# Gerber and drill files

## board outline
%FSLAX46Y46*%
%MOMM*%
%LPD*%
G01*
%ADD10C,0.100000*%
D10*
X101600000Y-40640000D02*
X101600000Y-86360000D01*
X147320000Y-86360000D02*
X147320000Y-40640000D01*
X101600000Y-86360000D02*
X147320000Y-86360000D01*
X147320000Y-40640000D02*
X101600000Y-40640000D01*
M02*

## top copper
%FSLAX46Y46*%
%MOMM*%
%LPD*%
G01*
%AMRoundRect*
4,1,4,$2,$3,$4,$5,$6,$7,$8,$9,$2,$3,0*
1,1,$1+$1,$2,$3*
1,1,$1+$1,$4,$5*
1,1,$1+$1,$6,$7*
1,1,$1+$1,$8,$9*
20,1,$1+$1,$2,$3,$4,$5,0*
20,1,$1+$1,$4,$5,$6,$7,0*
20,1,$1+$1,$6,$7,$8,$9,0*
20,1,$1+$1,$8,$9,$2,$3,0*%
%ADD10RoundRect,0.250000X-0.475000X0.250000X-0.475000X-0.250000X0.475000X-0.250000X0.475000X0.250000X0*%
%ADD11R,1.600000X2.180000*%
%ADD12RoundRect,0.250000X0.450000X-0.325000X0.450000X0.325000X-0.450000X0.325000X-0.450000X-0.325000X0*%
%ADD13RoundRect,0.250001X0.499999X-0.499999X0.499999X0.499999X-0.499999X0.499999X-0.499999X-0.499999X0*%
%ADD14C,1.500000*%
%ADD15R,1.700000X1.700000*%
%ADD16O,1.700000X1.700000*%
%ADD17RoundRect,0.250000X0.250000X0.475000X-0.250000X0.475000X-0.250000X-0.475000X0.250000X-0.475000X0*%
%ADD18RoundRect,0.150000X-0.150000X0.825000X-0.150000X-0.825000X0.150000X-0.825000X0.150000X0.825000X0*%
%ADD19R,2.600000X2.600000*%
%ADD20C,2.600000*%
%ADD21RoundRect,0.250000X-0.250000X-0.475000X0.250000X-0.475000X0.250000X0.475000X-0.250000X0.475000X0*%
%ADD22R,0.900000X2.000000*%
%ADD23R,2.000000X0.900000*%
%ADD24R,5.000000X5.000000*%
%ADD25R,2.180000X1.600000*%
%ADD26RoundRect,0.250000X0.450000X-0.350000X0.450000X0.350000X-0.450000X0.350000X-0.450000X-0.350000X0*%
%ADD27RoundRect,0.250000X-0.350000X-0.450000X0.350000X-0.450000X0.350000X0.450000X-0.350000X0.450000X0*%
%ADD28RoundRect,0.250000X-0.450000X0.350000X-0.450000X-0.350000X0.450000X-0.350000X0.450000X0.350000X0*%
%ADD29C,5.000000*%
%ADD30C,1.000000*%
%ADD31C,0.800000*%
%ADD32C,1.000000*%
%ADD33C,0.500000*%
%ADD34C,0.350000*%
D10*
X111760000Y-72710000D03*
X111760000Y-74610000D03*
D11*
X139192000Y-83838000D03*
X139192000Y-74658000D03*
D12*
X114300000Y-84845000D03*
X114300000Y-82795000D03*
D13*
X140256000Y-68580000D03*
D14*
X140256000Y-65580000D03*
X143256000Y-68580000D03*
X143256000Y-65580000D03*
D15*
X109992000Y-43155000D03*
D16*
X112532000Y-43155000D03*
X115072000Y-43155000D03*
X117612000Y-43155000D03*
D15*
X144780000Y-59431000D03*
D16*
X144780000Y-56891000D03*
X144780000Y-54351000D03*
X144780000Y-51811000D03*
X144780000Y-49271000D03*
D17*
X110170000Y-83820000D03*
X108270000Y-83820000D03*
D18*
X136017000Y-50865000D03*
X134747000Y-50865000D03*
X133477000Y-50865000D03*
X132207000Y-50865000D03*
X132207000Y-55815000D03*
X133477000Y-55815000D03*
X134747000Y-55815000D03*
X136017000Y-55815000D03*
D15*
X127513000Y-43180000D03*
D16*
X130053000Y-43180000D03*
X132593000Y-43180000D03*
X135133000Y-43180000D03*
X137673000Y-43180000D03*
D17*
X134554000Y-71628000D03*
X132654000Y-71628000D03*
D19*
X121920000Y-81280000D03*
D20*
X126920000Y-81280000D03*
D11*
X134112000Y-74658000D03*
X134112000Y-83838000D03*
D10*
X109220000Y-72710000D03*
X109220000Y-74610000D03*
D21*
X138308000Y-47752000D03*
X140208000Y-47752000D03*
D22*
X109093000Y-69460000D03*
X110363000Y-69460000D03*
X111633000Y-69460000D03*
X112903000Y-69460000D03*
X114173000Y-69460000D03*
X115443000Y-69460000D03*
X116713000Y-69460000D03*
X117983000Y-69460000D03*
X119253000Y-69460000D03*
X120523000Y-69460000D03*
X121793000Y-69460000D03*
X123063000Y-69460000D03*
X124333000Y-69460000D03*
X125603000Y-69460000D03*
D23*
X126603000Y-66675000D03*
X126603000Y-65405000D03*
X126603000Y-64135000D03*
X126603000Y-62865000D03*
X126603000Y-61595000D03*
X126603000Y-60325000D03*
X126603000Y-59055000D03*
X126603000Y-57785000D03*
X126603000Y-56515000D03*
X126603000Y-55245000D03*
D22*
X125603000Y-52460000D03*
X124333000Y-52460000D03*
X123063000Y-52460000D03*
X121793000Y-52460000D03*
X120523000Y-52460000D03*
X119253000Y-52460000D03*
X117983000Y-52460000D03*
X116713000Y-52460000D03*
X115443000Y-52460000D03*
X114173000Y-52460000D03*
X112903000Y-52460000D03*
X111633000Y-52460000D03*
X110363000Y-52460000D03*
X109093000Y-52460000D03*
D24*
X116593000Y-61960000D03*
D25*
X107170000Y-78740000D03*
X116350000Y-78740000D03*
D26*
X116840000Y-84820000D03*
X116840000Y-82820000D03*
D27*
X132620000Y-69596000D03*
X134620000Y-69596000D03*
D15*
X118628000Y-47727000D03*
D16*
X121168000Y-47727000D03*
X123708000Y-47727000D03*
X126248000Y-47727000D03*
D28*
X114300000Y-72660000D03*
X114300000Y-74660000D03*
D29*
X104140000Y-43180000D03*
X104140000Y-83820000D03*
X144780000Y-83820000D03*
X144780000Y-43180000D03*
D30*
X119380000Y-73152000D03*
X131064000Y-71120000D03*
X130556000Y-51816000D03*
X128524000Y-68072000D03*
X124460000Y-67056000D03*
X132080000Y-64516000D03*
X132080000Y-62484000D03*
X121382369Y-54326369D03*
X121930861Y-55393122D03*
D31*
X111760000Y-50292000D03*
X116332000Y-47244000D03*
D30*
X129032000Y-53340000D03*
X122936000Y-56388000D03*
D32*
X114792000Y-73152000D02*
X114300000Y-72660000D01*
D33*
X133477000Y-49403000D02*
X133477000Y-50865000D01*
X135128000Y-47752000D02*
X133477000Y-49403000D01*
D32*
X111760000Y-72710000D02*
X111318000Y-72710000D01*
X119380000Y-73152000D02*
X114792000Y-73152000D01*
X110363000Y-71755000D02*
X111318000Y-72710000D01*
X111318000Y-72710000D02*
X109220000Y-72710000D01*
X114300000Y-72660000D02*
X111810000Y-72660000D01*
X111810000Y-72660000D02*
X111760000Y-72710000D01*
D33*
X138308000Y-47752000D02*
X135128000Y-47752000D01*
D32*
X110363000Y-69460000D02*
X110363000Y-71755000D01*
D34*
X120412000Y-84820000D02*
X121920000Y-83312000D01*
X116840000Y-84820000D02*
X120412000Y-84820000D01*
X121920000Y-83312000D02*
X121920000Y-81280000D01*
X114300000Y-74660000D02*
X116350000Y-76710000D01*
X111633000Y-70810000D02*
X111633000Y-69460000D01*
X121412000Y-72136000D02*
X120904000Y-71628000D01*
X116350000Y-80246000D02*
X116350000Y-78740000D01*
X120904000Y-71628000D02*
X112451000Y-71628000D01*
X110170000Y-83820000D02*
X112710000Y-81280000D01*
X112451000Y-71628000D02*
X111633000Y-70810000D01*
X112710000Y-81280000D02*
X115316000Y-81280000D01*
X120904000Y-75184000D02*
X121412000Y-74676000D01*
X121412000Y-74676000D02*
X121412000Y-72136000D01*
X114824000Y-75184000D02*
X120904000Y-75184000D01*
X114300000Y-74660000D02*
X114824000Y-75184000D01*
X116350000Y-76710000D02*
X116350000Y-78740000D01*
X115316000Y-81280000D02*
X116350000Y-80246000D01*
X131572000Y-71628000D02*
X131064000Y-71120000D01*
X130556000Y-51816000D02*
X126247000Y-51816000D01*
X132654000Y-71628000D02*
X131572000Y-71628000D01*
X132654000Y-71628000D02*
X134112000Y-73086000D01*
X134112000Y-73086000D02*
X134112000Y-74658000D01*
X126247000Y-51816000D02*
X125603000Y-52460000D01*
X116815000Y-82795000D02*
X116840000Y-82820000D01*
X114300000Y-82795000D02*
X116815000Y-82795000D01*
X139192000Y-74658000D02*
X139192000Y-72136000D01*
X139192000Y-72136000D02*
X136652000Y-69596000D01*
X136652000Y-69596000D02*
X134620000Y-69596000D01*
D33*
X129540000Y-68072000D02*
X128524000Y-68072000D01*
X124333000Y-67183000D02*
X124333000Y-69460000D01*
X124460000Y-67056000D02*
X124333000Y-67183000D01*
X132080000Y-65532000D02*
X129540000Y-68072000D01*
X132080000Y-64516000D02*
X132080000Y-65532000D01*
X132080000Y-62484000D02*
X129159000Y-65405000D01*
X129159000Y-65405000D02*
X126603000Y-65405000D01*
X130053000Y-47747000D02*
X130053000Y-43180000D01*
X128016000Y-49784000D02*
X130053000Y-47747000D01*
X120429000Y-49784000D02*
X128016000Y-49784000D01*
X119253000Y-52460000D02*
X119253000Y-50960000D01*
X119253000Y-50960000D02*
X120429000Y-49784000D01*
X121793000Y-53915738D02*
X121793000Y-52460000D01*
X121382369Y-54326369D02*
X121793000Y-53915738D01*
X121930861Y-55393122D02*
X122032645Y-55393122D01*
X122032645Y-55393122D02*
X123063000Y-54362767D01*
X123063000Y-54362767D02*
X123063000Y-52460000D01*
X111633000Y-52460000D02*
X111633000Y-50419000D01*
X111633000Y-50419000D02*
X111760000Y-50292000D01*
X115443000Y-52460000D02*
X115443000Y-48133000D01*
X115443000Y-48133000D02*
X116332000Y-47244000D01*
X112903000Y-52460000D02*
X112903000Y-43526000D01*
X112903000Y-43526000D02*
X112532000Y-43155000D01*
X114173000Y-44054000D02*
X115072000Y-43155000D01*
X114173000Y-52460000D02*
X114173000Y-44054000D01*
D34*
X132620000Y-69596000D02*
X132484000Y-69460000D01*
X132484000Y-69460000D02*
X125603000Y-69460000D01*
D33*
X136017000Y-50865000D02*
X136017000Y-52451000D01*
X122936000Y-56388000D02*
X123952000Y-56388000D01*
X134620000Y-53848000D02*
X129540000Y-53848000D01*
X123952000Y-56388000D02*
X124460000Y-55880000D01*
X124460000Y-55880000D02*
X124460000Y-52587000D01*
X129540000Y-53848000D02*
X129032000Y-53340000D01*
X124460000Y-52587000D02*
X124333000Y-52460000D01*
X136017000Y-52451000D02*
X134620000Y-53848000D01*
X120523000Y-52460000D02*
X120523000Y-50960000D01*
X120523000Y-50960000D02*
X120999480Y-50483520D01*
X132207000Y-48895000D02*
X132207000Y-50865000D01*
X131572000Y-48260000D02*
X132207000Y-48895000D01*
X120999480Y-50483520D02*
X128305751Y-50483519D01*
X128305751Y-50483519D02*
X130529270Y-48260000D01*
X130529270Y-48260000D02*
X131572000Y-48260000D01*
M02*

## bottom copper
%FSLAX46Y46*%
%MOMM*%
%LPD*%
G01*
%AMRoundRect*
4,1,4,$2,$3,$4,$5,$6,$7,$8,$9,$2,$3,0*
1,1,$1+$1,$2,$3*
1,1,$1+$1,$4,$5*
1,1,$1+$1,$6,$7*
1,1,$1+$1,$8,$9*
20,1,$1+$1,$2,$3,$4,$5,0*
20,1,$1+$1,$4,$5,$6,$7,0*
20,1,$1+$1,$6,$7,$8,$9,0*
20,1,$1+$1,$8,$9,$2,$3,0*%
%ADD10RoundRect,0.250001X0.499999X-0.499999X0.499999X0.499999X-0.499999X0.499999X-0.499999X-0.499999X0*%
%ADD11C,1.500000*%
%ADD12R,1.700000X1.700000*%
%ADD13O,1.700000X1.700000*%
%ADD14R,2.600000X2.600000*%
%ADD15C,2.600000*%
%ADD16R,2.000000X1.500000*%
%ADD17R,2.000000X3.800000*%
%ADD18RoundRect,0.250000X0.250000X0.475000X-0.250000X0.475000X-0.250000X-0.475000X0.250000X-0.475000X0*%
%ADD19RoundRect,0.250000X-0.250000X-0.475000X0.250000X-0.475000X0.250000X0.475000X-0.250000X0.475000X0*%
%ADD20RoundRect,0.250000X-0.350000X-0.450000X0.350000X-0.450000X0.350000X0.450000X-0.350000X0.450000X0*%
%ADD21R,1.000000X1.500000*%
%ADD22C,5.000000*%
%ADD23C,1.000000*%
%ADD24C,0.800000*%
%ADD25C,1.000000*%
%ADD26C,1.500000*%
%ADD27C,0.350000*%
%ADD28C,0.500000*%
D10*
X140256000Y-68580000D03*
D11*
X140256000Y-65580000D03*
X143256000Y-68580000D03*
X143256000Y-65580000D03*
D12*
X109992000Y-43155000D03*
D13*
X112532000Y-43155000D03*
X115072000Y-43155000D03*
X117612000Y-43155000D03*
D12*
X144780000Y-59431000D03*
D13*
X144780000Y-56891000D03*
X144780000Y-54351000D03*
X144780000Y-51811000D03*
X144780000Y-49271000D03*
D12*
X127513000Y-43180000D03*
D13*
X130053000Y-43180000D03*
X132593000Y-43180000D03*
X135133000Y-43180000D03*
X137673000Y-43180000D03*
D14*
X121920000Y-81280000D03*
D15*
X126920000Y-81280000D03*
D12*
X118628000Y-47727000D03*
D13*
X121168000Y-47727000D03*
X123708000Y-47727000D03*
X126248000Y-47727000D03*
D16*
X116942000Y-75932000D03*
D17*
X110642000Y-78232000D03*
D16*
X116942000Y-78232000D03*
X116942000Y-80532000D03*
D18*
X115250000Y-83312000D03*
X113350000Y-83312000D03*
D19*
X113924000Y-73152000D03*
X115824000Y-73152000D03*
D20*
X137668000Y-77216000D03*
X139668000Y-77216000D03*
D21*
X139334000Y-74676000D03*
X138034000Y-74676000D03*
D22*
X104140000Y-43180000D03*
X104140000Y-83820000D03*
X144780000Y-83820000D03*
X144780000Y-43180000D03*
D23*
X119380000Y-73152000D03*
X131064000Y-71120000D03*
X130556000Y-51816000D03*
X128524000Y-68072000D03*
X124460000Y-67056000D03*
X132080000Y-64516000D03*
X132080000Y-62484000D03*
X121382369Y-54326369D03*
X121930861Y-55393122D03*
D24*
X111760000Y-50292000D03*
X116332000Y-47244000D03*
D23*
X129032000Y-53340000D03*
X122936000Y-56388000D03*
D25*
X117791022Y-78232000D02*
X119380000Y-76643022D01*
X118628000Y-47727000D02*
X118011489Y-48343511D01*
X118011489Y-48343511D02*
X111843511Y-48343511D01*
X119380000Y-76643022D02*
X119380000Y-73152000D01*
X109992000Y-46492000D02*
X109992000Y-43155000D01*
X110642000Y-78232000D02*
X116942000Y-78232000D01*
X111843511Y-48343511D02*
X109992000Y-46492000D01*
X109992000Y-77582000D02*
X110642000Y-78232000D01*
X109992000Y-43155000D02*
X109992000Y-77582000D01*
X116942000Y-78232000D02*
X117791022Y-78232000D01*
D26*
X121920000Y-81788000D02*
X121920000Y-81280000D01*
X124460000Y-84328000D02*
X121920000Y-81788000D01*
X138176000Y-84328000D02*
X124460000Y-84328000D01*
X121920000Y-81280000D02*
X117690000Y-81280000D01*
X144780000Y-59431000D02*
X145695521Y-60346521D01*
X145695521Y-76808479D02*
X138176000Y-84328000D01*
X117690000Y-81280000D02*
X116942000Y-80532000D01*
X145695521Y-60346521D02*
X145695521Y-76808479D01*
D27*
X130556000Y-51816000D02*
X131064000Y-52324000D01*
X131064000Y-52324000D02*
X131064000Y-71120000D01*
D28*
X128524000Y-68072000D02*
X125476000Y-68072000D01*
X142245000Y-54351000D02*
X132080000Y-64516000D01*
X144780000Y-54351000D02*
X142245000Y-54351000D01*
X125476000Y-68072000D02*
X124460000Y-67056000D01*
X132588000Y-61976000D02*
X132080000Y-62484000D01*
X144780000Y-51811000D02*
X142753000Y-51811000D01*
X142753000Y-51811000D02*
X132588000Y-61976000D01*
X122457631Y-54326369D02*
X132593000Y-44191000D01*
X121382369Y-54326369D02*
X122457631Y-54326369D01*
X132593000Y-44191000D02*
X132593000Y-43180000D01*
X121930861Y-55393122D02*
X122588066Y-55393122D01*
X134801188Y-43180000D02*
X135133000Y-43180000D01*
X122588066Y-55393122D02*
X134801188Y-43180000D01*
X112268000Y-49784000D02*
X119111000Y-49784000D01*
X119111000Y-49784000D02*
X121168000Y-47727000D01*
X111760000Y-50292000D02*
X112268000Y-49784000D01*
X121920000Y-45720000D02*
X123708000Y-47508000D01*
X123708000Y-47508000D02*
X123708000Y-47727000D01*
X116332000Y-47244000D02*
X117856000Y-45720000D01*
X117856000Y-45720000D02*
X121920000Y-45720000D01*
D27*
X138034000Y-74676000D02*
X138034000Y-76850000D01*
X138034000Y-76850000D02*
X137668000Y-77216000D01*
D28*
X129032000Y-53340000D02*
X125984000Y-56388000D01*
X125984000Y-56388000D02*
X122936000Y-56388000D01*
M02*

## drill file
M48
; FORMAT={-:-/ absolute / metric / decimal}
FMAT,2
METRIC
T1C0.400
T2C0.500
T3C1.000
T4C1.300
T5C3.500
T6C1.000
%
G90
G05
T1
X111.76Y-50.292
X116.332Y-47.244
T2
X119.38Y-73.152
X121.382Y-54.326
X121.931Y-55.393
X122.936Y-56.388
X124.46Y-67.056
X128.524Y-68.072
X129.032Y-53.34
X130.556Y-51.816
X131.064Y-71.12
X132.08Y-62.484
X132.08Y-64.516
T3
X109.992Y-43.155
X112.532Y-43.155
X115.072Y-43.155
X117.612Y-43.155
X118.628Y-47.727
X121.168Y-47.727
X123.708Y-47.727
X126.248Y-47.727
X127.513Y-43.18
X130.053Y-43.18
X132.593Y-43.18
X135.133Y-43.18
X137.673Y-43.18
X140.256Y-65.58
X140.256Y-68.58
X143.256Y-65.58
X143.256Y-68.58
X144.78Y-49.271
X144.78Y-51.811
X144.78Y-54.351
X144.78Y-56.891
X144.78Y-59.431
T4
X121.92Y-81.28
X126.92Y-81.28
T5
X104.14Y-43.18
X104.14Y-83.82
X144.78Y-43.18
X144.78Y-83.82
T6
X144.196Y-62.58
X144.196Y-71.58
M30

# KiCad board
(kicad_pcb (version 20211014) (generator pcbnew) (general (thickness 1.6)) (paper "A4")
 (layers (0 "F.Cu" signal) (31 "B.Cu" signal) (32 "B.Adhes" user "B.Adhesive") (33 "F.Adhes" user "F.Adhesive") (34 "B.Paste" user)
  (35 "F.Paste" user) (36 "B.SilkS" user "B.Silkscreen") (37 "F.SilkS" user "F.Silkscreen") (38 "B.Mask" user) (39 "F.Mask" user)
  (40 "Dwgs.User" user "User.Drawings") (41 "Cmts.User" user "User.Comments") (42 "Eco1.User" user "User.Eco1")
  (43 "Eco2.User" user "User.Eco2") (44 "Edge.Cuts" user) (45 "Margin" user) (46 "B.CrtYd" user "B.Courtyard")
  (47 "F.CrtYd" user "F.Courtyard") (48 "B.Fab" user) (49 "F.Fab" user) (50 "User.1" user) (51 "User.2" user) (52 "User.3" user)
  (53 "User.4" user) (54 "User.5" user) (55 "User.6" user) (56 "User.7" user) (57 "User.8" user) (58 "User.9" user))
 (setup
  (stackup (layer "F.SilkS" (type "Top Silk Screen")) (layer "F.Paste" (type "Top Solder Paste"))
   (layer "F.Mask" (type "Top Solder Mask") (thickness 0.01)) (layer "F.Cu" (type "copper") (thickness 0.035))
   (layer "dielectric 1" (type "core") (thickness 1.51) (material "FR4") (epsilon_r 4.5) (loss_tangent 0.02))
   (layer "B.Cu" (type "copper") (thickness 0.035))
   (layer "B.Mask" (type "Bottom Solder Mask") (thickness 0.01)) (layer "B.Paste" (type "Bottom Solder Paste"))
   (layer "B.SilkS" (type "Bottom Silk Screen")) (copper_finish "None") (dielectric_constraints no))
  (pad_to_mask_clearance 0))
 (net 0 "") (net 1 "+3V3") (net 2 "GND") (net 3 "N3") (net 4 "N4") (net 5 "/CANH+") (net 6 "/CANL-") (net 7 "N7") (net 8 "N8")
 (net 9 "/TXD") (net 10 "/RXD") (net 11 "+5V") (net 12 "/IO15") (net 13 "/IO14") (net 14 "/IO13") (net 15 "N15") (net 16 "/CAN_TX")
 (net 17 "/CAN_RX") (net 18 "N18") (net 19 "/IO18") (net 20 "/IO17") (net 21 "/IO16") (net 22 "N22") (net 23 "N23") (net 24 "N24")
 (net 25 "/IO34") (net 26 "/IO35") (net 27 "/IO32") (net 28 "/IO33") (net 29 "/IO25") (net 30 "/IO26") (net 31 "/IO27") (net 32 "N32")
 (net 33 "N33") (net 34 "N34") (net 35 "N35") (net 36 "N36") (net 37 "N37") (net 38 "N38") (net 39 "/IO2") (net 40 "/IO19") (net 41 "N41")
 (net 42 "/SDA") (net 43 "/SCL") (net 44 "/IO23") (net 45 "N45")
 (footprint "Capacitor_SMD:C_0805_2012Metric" (layer "F.Cu") (at 111.76 73.66 -90)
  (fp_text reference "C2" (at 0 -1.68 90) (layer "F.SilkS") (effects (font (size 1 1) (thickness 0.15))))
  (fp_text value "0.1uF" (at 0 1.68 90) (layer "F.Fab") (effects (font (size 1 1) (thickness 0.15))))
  (pad "1" smd roundrect (at -0.95 0 270) (size 1 1.45) (layers "F.Cu" "F.Paste" "F.Mask") (roundrect_rratio 0.25) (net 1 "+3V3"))
  (pad "2" smd roundrect (at 0.95 0 270) (size 1 1.45) (layers "F.Cu" "F.Paste" "F.Mask") (roundrect_rratio 0.25) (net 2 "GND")))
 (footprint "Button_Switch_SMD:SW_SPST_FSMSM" (layer "F.Cu") (at 139.192 79.248 90)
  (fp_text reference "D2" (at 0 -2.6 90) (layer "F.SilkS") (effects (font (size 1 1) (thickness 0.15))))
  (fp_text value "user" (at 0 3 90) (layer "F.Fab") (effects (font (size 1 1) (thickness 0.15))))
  (pad "1" smd rect (at -4.59 0 90) (size 2.18 1.6) (layers "F.Cu" "F.Paste" "F.Mask") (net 2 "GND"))
  (pad "2" smd rect (at 4.59 0 90) (size 2.18 1.6) (layers "F.Cu" "F.Paste" "F.Mask") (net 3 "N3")))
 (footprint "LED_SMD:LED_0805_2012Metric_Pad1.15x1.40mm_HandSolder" (layer "F.Cu") (at 114.3 83.82 90)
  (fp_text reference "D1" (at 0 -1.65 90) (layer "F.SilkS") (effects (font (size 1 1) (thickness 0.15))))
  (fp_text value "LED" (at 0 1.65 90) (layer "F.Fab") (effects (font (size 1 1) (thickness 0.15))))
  (pad "1" smd roundrect (at -1.025 0 90) (size 1.15 1.4) (layers "F.Cu" "F.Paste" "F.Mask") (roundrect_rratio 0.217391) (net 2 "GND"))
  (pad "2" smd roundrect (at 1.025 0 90) (size 1.15 1.4) (layers "F.Cu" "F.Paste" "F.Mask") (roundrect_rratio 0.217391) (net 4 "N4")))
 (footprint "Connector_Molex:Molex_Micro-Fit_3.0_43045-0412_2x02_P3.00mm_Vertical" (layer "F.Cu") (at 140.256 68.58 90)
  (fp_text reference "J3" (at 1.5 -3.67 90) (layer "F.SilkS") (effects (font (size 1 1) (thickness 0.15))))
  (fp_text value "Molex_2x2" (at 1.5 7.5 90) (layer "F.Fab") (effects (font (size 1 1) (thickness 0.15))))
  (pad "" np_thru_hole circle (at -3 3.94 90) (size 1 1) (drill 1) (layers *.Cu *.Mask))
  (pad "" np_thru_hole circle (at 6 3.94 90) (size 1 1) (drill 1) (layers *.Cu *.Mask))
  (pad "1" thru_hole roundrect (at 0 0 90) (size 1.5 1.5) (drill 1) (layers *.Cu *.Mask) (roundrect_rratio 0.166667) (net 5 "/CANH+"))
  (pad "2" thru_hole circle (at 3 0 90) (size 1.5 1.5) (drill 1) (layers *.Cu *.Mask) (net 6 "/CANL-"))
  (pad "3" thru_hole circle (at 0 3 90) (size 1.5 1.5) (drill 1) (layers *.Cu *.Mask) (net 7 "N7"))
  (pad "4" thru_hole circle (at 3 3 90) (size 1.5 1.5) (drill 1) (layers *.Cu *.Mask) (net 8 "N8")))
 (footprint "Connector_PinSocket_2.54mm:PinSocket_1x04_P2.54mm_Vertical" (layer "F.Cu") (at 109.992 43.155 90)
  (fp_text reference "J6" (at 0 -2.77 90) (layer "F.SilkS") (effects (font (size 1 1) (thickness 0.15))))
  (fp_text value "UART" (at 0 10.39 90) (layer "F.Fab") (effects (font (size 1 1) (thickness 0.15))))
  (pad "1" thru_hole rect (at 0 0 90) (size 1.7 1.7) (drill 1) (layers *.Cu *.Mask) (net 1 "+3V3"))
  (pad "2" thru_hole oval (at 0 2.54 90) (size 1.7 1.7) (drill 1) (layers *.Cu *.Mask) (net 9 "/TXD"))
  (pad "3" thru_hole oval (at 0 5.08 90) (size 1.7 1.7) (drill 1) (layers *.Cu *.Mask) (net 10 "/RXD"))
  (pad "4" thru_hole oval (at 0 7.62 90) (size 1.7 1.7) (drill 1) (layers *.Cu *.Mask) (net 2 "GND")))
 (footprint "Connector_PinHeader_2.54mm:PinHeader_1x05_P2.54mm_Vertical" (layer "F.Cu") (at 144.78 59.431 180)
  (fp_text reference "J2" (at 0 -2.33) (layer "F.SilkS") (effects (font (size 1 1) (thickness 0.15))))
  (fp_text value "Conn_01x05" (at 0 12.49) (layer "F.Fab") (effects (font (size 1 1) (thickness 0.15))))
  (pad "1" thru_hole rect (at 0 0 180) (size 1.7 1.7) (drill 1) (layers *.Cu *.Mask) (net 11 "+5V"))
  (pad "2" thru_hole oval (at 0 2.54 180) (size 1.7 1.7) (drill 1) (layers *.Cu *.Mask) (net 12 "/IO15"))
  (pad "3" thru_hole oval (at 0 5.08 180) (size 1.7 1.7) (drill 1) (layers *.Cu *.Mask) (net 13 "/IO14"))
  (pad "4" thru_hole oval (at 0 7.62 180) (size 1.7 1.7) (drill 1) (layers *.Cu *.Mask) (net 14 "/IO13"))
  (pad "5" thru_hole oval (at 0 10.16 180) (size 1.7 1.7) (drill 1) (layers *.Cu *.Mask) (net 2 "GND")))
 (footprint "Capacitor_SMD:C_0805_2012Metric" (layer "F.Cu") (at 109.22 83.82 180)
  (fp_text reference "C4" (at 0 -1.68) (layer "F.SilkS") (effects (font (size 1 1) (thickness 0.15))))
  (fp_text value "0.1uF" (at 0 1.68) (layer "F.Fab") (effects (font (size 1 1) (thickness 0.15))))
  (pad "1" smd roundrect (at -0.95 0 180) (size 1 1.45) (layers "F.Cu" "F.Paste" "F.Mask") (roundrect_rratio 0.25) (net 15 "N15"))
  (pad "2" smd roundrect (at 0.95 0 180) (size 1 1.45) (layers "F.Cu" "F.Paste" "F.Mask") (roundrect_rratio 0.25) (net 2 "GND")))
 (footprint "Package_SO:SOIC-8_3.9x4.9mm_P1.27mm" (layer "F.Cu") (at 134.112 53.34 -90)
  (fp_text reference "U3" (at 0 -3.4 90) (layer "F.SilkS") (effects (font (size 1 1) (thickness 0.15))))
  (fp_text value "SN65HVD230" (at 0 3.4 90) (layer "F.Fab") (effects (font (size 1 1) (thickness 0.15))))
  (pad "1" smd roundrect (at -2.475 -1.905 270) (size 1.95 0.6) (layers "F.Cu" "F.Paste" "F.Mask") (roundrect_rratio 0.25)
   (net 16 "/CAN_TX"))
  (pad "2" smd roundrect (at -2.475 -0.635 270) (size 1.95 0.6) (layers "F.Cu" "F.Paste" "F.Mask") (roundrect_rratio 0.25) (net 2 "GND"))
  (pad "3" smd roundrect (at -2.475 0.635 270) (size 1.95 0.6) (layers "F.Cu" "F.Paste" "F.Mask") (roundrect_rratio 0.25) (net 1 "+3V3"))
  (pad "4" smd roundrect (at -2.475 1.905 270) (size 1.95 0.6) (layers "F.Cu" "F.Paste" "F.Mask") (roundrect_rratio 0.25) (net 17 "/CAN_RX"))
  (pad "5" smd roundrect (at 2.475 1.905 270) (size 1.95 0.6) (layers "F.Cu" "F.Paste" "F.Mask") (roundrect_rratio 0.25) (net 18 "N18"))
  (pad "6" smd roundrect (at 2.475 0.635 270) (size 1.95 0.6) (layers "F.Cu" "F.Paste" "F.Mask") (roundrect_rratio 0.25) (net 5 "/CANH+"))
  (pad "7" smd roundrect (at 2.475 -0.635 270) (size 1.95 0.6) (layers "F.Cu" "F.Paste" "F.Mask") (roundrect_rratio 0.25) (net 6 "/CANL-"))
  (pad "8" smd roundrect (at 2.475 -1.905 270) (size 1.95 0.6) (layers "F.Cu" "F.Paste" "F.Mask") (roundrect_rratio 0.25) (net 2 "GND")))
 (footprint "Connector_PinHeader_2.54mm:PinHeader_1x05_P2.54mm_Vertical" (layer "F.Cu") (at 127.513 43.18 90)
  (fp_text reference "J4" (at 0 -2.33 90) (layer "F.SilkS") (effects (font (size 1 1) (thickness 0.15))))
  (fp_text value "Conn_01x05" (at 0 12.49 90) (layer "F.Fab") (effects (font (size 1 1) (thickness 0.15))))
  (pad "1" thru_hole rect (at 0 0 90) (size 1.7 1.7) (drill 1) (layers *.Cu *.Mask) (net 11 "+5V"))
  (pad "2" thru_hole oval (at 0 2.54 90) (size 1.7 1.7) (drill 1) (layers *.Cu *.Mask) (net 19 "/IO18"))
  (pad "3" thru_hole oval (at 0 5.08 90) (size 1.7 1.7) (drill 1) (layers *.Cu *.Mask) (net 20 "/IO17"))
  (pad "4" thru_hole oval (at 0 7.62 90) (size 1.7 1.7) (drill 1) (layers *.Cu *.Mask) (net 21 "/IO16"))
  (pad "5" thru_hole oval (at 0 10.16 90) (size 1.7 1.7) (drill 1) (layers *.Cu *.Mask) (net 2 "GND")))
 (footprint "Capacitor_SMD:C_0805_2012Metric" (layer "F.Cu") (at 133.604 71.628 180)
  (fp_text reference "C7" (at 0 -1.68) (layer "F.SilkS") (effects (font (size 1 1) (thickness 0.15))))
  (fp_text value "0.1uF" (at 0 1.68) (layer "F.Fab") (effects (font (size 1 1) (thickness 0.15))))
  (pad "1" smd roundrect (at -0.95 0 180) (size 1 1.45) (layers "F.Cu" "F.Paste" "F.Mask") (roundrect_rratio 0.25) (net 2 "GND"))
  (pad "2" smd roundrect (at 0.95 0 180) (size 1 1.45) (layers "F.Cu" "F.Paste" "F.Mask") (roundrect_rratio 0.25) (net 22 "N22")))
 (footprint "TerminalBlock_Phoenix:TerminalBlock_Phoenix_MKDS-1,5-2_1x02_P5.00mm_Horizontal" (layer "F.Cu") (at 121.92 81.28)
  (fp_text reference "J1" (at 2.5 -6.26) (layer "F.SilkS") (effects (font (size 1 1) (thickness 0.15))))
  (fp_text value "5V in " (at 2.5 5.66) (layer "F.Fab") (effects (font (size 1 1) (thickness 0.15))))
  (pad "1" thru_hole rect (at 0 0) (size 2.6 2.6) (drill 1.3) (layers *.Cu *.Mask) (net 11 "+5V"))
  (pad "2" thru_hole circle (at 5 0) (size 2.6 2.6) (drill 1.3) (layers *.Cu *.Mask) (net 2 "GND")))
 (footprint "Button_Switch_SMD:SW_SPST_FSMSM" (layer "F.Cu") (at 134.112 79.248 -90)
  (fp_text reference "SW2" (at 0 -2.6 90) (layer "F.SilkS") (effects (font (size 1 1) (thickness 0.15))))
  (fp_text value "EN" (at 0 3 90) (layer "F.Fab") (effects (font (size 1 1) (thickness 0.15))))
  (pad "1" smd rect (at -4.59 0 270) (size 2.18 1.6) (layers "F.Cu" "F.Paste" "F.Mask") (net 22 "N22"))
  (pad "2" smd rect (at 4.59 0 270) (size 2.18 1.6) (layers "F.Cu" "F.Paste" "F.Mask") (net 2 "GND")))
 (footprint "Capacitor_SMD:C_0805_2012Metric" (layer "F.Cu") (at 109.22 73.66 -90)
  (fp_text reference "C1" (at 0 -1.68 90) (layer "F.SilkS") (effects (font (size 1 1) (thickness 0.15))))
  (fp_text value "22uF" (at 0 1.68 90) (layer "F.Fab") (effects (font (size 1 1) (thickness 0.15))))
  (pad "1" smd roundrect (at -0.95 0 270) (size 1 1.45) (layers "F.Cu" "F.Paste" "F.Mask") (roundrect_rratio 0.25) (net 1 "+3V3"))
  (pad "2" smd roundrect (at 0.95 0 270) (size 1 1.45) (layers "F.Cu" "F.Paste" "F.Mask") (roundrect_rratio 0.25) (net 2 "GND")))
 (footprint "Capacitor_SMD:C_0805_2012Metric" (layer "F.Cu") (at 139.258 47.752)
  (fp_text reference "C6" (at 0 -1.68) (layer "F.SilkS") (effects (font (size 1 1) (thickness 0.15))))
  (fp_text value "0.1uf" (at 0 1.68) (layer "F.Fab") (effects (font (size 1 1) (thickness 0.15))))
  (pad "1" smd roundrect (at -0.95 0) (size 1 1.45) (layers "F.Cu" "F.Paste" "F.Mask") (roundrect_rratio 0.25) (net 1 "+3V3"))
  (pad "2" smd roundrect (at 0.95 0) (size 1 1.45) (layers "F.Cu" "F.Paste" "F.Mask") (roundrect_rratio 0.25) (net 2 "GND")))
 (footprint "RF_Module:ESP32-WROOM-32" (layer "F.Cu") (at 117.348 60.96 90)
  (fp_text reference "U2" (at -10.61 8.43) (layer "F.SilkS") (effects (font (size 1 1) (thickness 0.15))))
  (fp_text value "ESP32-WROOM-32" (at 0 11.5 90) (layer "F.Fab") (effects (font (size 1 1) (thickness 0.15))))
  (pad "1" smd rect (at -8.5 -8.255 90) (size 2 0.9) (layers "F.Cu" "F.Paste" "F.Mask") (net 2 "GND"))
  (pad "2" smd rect (at -8.5 -6.985 90) (size 2 0.9) (layers "F.Cu" "F.Paste" "F.Mask") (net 1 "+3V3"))
  (pad "3" smd rect (at -8.5 -5.715 90) (size 2 0.9) (layers "F.Cu" "F.Paste" "F.Mask") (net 15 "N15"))
  (pad "4" smd rect (at -8.5 -4.445 90) (size 2 0.9) (layers "F.Cu" "F.Paste" "F.Mask") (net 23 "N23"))
  (pad "5" smd rect (at -8.5 -3.175 90) (size 2 0.9) (layers "F.Cu" "F.Paste" "F.Mask") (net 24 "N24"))
  (pad "6" smd rect (at -8.5 -1.905 90) (size 2 0.9) (layers "F.Cu" "F.Paste" "F.Mask") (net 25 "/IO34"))
  (pad "7" smd rect (at -8.5 -0.635 90) (size 2 0.9) (layers "F.Cu" "F.Paste" "F.Mask") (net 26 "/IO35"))
  (pad "8" smd rect (at -8.5 0.635 90) (size 2 0.9) (layers "F.Cu" "F.Paste" "F.Mask") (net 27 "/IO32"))
  (pad "9" smd rect (at -8.5 1.905 90) (size 2 0.9) (layers "F.Cu" "F.Paste" "F.Mask") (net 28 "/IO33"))
  (pad "10" smd rect (at -8.5 3.175 90) (size 2 0.9) (layers "F.Cu" "F.Paste" "F.Mask") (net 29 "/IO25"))
  (pad "11" smd rect (at -8.5 4.445 90) (size 2 0.9) (layers "F.Cu" "F.Paste" "F.Mask") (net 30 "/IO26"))
  (pad "12" smd rect (at -8.5 5.715 90) (size 2 0.9) (layers "F.Cu" "F.Paste" "F.Mask") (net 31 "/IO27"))
  (pad "13" smd rect (at -8.5 6.985 90) (size 2 0.9) (layers "F.Cu" "F.Paste" "F.Mask") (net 13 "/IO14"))
  (pad "14" smd rect (at -8.5 8.255 90) (size 2 0.9) (layers "F.Cu" "F.Paste" "F.Mask") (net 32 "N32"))
  (pad "15" smd rect (at -5.715 9.255 180) (size 2 0.9) (layers "F.Cu" "F.Paste" "F.Mask") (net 2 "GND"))
  (pad "16" smd rect (at -4.445 9.255 180) (size 2 0.9) (layers "F.Cu" "F.Paste" "F.Mask") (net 14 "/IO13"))
  (pad "17" smd rect (at -3.175 9.255 180) (size 2 0.9) (layers "F.Cu" "F.Paste" "F.Mask") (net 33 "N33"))
  (pad "18" smd rect (at -1.905 9.255 180) (size 2 0.9) (layers "F.Cu" "F.Paste" "F.Mask") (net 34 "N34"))
  (pad "19" smd rect (at -0.635 9.255 180) (size 2 0.9) (layers "F.Cu" "F.Paste" "F.Mask") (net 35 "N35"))
  (pad "20" smd rect (at 0.635 9.255 180) (size 2 0.9) (layers "F.Cu" "F.Paste" "F.Mask") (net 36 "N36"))
  (pad "21" smd rect (at 1.905 9.255 180) (size 2 0.9) (layers "F.Cu" "F.Paste" "F.Mask") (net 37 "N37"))
  (pad "22" smd rect (at 3.175 9.255 180) (size 2 0.9) (layers "F.Cu" "F.Paste" "F.Mask") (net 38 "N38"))
  (pad "23" smd rect (at 4.445 9.255 180) (size 2 0.9) (layers "F.Cu" "F.Paste" "F.Mask") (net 12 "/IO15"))
  (pad "24" smd rect (at 5.715 9.255 180) (size 2 0.9) (layers "F.Cu" "F.Paste" "F.Mask") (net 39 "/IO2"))
  (pad "25" smd rect (at 8.5 8.255 90) (size 2 0.9) (layers "F.Cu" "F.Paste" "F.Mask") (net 22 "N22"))
  (pad "26" smd rect (at 8.5 6.985 90) (size 2 0.9) (layers "F.Cu" "F.Paste" "F.Mask") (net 16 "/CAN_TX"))
  (pad "27" smd rect (at 8.5 5.715 90) (size 2 0.9) (layers "F.Cu" "F.Paste" "F.Mask") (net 21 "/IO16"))
  (pad "28" smd rect (at 8.5 4.445 90) (size 2 0.9) (layers "F.Cu" "F.Paste" "F.Mask") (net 20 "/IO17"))
  (pad "29" smd rect (at 8.5 3.175 90) (size 2 0.9) (layers "F.Cu" "F.Paste" "F.Mask") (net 17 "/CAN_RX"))
  (pad "30" smd rect (at 8.5 1.905 90) (size 2 0.9) (layers "F.Cu" "F.Paste" "F.Mask") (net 19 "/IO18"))
  (pad "31" smd rect (at 8.5 0.635 90) (size 2 0.9) (layers "F.Cu" "F.Paste" "F.Mask") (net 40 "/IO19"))
  (pad "32" smd rect (at 8.5 -0.635 90) (size 2 0.9) (layers "F.Cu" "F.Paste" "F.Mask") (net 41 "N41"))
  (pad "33" smd rect (at 8.5 -1.905 90) (size 2 0.9) (layers "F.Cu" "F.Paste" "F.Mask") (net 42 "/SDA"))
  (pad "34" smd rect (at 8.5 -3.175 90) (size 2 0.9) (layers "F.Cu" "F.Paste" "F.Mask") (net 10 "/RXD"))
  (pad "35" smd rect (at 8.5 -4.445 90) (size 2 0.9) (layers "F.Cu" "F.Paste" "F.Mask") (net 9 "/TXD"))
  (pad "36" smd rect (at 8.5 -5.715 90) (size 2 0.9) (layers "F.Cu" "F.Paste" "F.Mask") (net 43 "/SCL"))
  (pad "37" smd rect (at 8.5 -6.985 90) (size 2 0.9) (layers "F.Cu" "F.Paste" "F.Mask") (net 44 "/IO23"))
  (pad "38" smd rect (at 8.5 -8.255 90) (size 2 0.9) (layers "F.Cu" "F.Paste" "F.Mask") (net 2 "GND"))
  (pad "39" smd rect (at -1 -0.755 90) (size 5 5) (layers "F.Cu" "F.Paste" "F.Mask") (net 2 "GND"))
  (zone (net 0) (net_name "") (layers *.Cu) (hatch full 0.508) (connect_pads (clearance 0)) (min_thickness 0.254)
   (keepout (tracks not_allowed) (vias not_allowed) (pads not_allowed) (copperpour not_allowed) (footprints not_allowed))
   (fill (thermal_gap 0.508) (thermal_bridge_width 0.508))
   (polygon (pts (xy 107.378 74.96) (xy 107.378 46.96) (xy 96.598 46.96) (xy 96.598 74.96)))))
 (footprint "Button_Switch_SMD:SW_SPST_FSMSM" (layer "F.Cu") (at 111.76 78.74)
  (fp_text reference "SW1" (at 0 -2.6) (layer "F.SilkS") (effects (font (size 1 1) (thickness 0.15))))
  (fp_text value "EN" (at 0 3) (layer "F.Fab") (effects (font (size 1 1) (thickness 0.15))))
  (pad "1" smd rect (at -4.59 0) (size 2.18 1.6) (layers "F.Cu" "F.Paste" "F.Mask") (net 2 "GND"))
  (pad "2" smd rect (at 4.59 0) (size 2.18 1.6) (layers "F.Cu" "F.Paste" "F.Mask") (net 15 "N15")))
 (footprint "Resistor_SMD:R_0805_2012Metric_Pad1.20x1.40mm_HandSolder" (layer "F.Cu") (at 116.84 83.82 90)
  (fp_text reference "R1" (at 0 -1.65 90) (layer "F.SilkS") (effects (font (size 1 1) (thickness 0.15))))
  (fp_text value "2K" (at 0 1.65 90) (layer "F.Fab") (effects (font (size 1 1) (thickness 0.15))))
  (pad "1" smd roundrect (at -1 0 90) (size 1.2 1.4) (layers "F.Cu" "F.Paste" "F.Mask") (roundrect_rratio 0.208333) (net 11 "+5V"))
  (pad "2" smd roundrect (at 1 0 90) (size 1.2 1.4) (layers "F.Cu" "F.Paste" "F.Mask") (roundrect_rratio 0.208333) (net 4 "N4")))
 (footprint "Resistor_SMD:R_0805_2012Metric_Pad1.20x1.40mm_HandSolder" (layer "F.Cu") (at 133.62 69.596)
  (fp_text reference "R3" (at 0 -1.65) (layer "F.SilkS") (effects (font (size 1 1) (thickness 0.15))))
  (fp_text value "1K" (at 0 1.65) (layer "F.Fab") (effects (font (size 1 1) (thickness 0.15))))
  (pad "1" smd roundrect (at -1 0) (size 1.2 1.4) (layers "F.Cu" "F.Paste" "F.Mask") (roundrect_rratio 0.208333) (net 32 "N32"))
  (pad "2" smd roundrect (at 1 0) (size 1.2 1.4) (layers "F.Cu" "F.Paste" "F.Mask") (roundrect_rratio 0.208333) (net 3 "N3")))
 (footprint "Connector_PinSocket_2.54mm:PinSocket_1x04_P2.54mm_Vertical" (layer "F.Cu") (at 118.628 47.727 90)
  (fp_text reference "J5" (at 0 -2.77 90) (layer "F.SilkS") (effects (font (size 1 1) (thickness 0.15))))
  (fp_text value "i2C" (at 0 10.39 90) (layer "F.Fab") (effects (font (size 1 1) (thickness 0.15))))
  (pad "1" thru_hole rect (at 0 0 90) (size 1.7 1.7) (drill 1) (layers *.Cu *.Mask) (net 1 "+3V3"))
  (pad "2" thru_hole oval (at 0 2.54 90) (size 1.7 1.7) (drill 1) (layers *.Cu *.Mask) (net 43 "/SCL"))
  (pad "3" thru_hole oval (at 0 5.08 90) (size 1.7 1.7) (drill 1) (layers *.Cu *.Mask) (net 42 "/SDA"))
  (pad "4" thru_hole oval (at 0 7.62 90) (size 1.7 1.7) (drill 1) (layers *.Cu *.Mask) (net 2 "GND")))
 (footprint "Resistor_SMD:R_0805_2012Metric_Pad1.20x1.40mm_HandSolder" (layer "F.Cu") (at 114.3 73.66 -90)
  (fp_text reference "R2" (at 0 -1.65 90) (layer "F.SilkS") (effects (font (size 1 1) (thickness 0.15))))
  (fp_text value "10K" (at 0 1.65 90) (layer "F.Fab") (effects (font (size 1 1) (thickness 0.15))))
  (pad "1" smd roundrect (at -1 0 270) (size 1.2 1.4) (layers "F.Cu" "F.Paste" "F.Mask") (roundrect_rratio 0.208333) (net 1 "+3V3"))
  (pad "2" smd roundrect (at 1 0 270) (size 1.2 1.4) (layers "F.Cu" "F.Paste" "F.Mask") (roundrect_rratio 0.208333) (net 15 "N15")))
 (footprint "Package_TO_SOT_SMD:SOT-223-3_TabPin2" (layer "B.Cu") (at 113.792 78.232 180)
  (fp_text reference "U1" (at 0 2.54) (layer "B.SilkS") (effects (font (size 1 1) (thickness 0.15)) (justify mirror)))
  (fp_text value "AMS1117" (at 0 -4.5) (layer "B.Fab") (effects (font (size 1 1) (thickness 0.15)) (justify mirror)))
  (pad "1" smd rect (at -3.15 2.3 180) (size 2 1.5) (layers "B.Cu" "B.Paste" "B.Mask") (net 2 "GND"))
  (pad "2" smd rect (at 3.15 0 180) (size 2 3.8) (layers "B.Cu" "B.Paste" "B.Mask") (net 1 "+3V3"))
  (pad "2" smd rect (at -3.15 0 180) (size 2 1.5) (layers "B.Cu" "B.Paste" "B.Mask") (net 1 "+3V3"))
  (pad "3" smd rect (at -3.15 -2.3 180) (size 2 1.5) (layers "B.Cu" "B.Paste" "B.Mask") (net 11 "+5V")))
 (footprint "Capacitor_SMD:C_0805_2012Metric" (layer "B.Cu") (at 114.3 83.312 180)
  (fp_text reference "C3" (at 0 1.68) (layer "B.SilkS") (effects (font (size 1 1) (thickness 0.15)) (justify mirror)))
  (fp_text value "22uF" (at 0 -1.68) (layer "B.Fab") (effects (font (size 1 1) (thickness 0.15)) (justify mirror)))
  (pad "1" smd roundrect (at -0.95 0 180) (size 1 1.45) (layers "B.Cu" "B.Paste" "B.Mask") (roundrect_rratio 0.25) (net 11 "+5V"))
  (pad "2" smd roundrect (at 0.95 0 180) (size 1 1.45) (layers "B.Cu" "B.Paste" "B.Mask") (roundrect_rratio 0.25) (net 2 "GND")))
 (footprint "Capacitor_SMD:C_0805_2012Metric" (layer "B.Cu") (at 114.874 73.152)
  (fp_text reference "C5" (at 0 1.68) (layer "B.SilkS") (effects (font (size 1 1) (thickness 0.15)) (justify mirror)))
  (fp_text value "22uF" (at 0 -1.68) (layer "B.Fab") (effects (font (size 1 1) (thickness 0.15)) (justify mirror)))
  (pad "1" smd roundrect (at -0.95 0) (size 1 1.45) (layers "B.Cu" "B.Paste" "B.Mask") (roundrect_rratio 0.25) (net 1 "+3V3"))
  (pad "2" smd roundrect (at 0.95 0) (size 1 1.45) (layers "B.Cu" "B.Paste" "B.Mask") (roundrect_rratio 0.25) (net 2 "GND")))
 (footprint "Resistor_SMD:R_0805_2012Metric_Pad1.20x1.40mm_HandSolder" (layer "B.Cu") (at 138.668 77.216)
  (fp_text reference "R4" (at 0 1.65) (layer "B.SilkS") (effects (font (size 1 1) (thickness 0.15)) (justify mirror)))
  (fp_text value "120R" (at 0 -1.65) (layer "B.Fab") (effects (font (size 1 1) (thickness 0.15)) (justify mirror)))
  (pad "1" smd roundrect (at -1 0) (size 1.2 1.4) (layers "B.Cu" "B.Paste" "B.Mask") (roundrect_rratio 0.208333) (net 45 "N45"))
  (pad "2" smd roundrect (at 1 0) (size 1.2 1.4) (layers "B.Cu" "B.Paste" "B.Mask") (roundrect_rratio 0.208333) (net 6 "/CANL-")))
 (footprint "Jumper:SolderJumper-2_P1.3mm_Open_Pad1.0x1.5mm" (layer "B.Cu") (at 138.684 74.676 180)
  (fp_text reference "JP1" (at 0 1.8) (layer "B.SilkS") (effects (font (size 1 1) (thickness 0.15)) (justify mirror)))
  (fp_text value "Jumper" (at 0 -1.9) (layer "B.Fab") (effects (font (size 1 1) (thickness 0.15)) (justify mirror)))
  (pad "1" smd rect (at -0.65 0 180) (size 1 1.5) (layers "B.Cu" "B.Mask") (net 5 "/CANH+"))
  (pad "2" smd rect (at 0.65 0 180) (size 1 1.5) (layers "B.Cu" "B.Mask") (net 45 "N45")))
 (gr_line (start 101.6 40.64) (end 101.6 86.36) (layer "Edge.Cuts") (width 0.1))
 (gr_line (start 147.32 86.36) (end 147.32 40.64) (layer "Edge.Cuts") (width 0.1))
 (gr_line (start 101.6 86.36) (end 147.32 86.36) (layer "Edge.Cuts") (width 0.1))
 (gr_line (start 147.32 40.64) (end 101.6 40.64) (layer "Edge.Cuts") (width 0.1))
 (via (at 104.14 43.18) (size 5) (drill 3.5) (layers "F.Cu" "B.Cu") (free) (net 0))
 (via (at 104.14 83.82) (size 5) (drill 3.5) (layers "F.Cu" "B.Cu") (free) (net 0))
 (via (at 144.78 83.82) (size 5) (drill 3.5) (layers "F.Cu" "B.Cu") (free) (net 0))
 (via (at 144.78 43.18) (size 5) (drill 3.5) (layers "F.Cu" "B.Cu") (free) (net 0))
 (segment (start 114.792 73.152) (end 114.3 72.66) (width 1) (layer "F.Cu") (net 1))
 (segment (start 133.477 49.403) (end 133.477 50.865) (width 0.5) (layer "F.Cu") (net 1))
 (segment (start 135.128 47.752) (end 133.477 49.403) (width 0.5) (layer "F.Cu") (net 1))
 (segment (start 111.76 72.71) (end 111.318 72.71) (width 1) (layer "F.Cu") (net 1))
 (segment (start 119.38 73.152) (end 114.792 73.152) (width 1) (layer "F.Cu") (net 1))
 (segment (start 110.363 71.755) (end 111.318 72.71) (width 1) (layer "F.Cu") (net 1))
 (segment (start 111.318 72.71) (end 109.22 72.71) (width 1) (layer "F.Cu") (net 1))
 (segment (start 114.3 72.66) (end 111.81 72.66) (width 1) (layer "F.Cu") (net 1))
 (segment (start 111.81 72.66) (end 111.76 72.71) (width 1) (layer "F.Cu") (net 1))
 (segment (start 138.308 47.752) (end 135.128 47.752) (width 0.5) (layer "F.Cu") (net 1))
 (segment (start 110.363 69.46) (end 110.363 71.755) (width 1) (layer "F.Cu") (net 1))
 (via (at 119.38 73.152) (size 1) (drill 0.5) (layers "F.Cu" "B.Cu") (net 1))
 (segment (start 117.791022 78.232) (end 119.38 76.643022) (width 1) (layer "B.Cu") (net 1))
 (segment (start 118.628 47.727) (end 118.011489 48.343511) (width 1) (layer "B.Cu") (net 1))
 (segment (start 118.011489 48.343511) (end 111.843511 48.343511) (width 1) (layer "B.Cu") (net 1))
 (segment (start 119.38 76.643022) (end 119.38 73.152) (width 1) (layer "B.Cu") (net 1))
 (segment (start 109.992 46.492) (end 109.992 43.155) (width 1) (layer "B.Cu") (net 1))
 (segment (start 110.642 78.232) (end 116.942 78.232) (width 1) (layer "B.Cu") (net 1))
 (segment (start 111.843511 48.343511) (end 109.992 46.492) (width 1) (layer "B.Cu") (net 1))
 (segment (start 109.992 77.582) (end 110.642 78.232) (width 1) (layer "B.Cu") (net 1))
 (segment (start 109.992 43.155) (end 109.992 77.582) (width 1) (layer "B.Cu") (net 1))
 (segment (start 116.942 78.232) (end 117.791022 78.232) (width 1) (layer "B.Cu") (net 1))
 (segment (start 120.412 84.82) (end 121.92 83.312) (width 0.35) (layer "F.Cu") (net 11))
 (segment (start 116.84 84.82) (end 120.412 84.82) (width 0.35) (layer "F.Cu") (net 11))
 (segment (start 121.92 83.312) (end 121.92 81.28) (width 0.35) (layer "F.Cu") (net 11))
 (segment (start 121.92 81.788) (end 121.92 81.28) (width 1.5) (layer "B.Cu") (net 11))
 (segment (start 124.46 84.328) (end 121.92 81.788) (width 1.5) (layer "B.Cu") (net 11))
 (segment (start 138.176 84.328) (end 124.46 84.328) (width 1.5) (layer "B.Cu") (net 11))
 (segment (start 121.92 81.28) (end 117.69 81.28) (width 1.5) (layer "B.Cu") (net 11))
 (segment (start 144.78 59.431) (end 145.695521 60.346521) (width 1.5) (layer "B.Cu") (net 11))
 (segment (start 145.695521 76.808479) (end 138.176 84.328) (width 1.5) (layer "B.Cu") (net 11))
 (segment (start 117.69 81.28) (end 116.942 80.532) (width 1.5) (layer "B.Cu") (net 11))
 (segment (start 145.695521 60.346521) (end 145.695521 76.808479) (width 1.5) (layer "B.Cu") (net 11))
 (segment (start 114.3 74.66) (end 116.35 76.71) (width 0.35) (layer "F.Cu") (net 15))
 (segment (start 111.633 70.81) (end 111.633 69.46) (width 0.35) (layer "F.Cu") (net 15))
 (segment (start 121.412 72.136) (end 120.904 71.628) (width 0.35) (layer "F.Cu") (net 15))
 (segment (start 116.35 80.246) (end 116.35 78.74) (width 0.35) (layer "F.Cu") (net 15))
 (segment (start 120.904 71.628) (end 112.451 71.628) (width 0.35) (layer "F.Cu") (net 15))
 (segment (start 110.17 83.82) (end 112.71 81.28) (width 0.35) (layer "F.Cu") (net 15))
 (segment (start 112.451 71.628) (end 111.633 70.81) (width 0.35) (layer "F.Cu") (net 15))
 (segment (start 112.71 81.28) (end 115.316 81.28) (width 0.35) (layer "F.Cu") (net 15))
 (segment (start 120.904 75.184) (end 121.412 74.676) (width 0.35) (layer "F.Cu") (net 15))
 (segment (start 121.412 74.676) (end 121.412 72.136) (width 0.35) (layer "F.Cu") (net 15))
 (segment (start 114.824 75.184) (end 120.904 75.184) (width 0.35) (layer "F.Cu") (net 15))
 (segment (start 114.3 74.66) (end 114.824 75.184) (width 0.35) (layer "F.Cu") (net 15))
 (segment (start 116.35 76.71) (end 116.35 78.74) (width 0.35) (layer "F.Cu") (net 15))
 (segment (start 115.316 81.28) (end 116.35 80.246) (width 0.35) (layer "F.Cu") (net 15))
 (segment (start 131.572 71.628) (end 131.064 71.12) (width 0.35) (layer "F.Cu") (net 22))
 (segment (start 130.556 51.816) (end 126.247 51.816) (width 0.35) (layer "F.Cu") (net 22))
 (segment (start 132.654 71.628) (end 131.572 71.628) (width 0.35) (layer "F.Cu") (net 22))
 (segment (start 132.654 71.628) (end 134.112 73.086) (width 0.35) (layer "F.Cu") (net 22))
 (segment (start 134.112 73.086) (end 134.112 74.658) (width 0.35) (layer "F.Cu") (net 22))
 (segment (start 126.247 51.816) (end 125.603 52.46) (width 0.35) (layer "F.Cu") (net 22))
 (via (at 131.064 71.12) (size 1) (drill 0.5) (layers "F.Cu" "B.Cu") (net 22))
 (via (at 130.556 51.816) (size 1) (drill 0.5) (layers "F.Cu" "B.Cu") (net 22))
 (segment (start 130.556 51.816) (end 131.064 52.324) (width 0.35) (layer "B.Cu") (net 22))
 (segment (start 131.064 52.324) (end 131.064 71.12) (width 0.35) (layer "B.Cu") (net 22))
 (segment (start 116.815 82.795) (end 116.84 82.82) (width 0.35) (layer "F.Cu") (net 4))
 (segment (start 114.3 82.795) (end 116.815 82.795) (width 0.35) (layer "F.Cu") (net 4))
 (segment (start 139.192 74.658) (end 139.192 72.136) (width 0.35) (layer "F.Cu") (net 3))
 (segment (start 139.192 72.136) (end 136.652 69.596) (width 0.35) (layer "F.Cu") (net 3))
 (segment (start 136.652 69.596) (end 134.62 69.596) (width 0.35) (layer "F.Cu") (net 3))
 (segment (start 129.54 68.072) (end 128.524 68.072) (width 0.5) (layer "F.Cu") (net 13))
 (segment (start 124.333 67.183) (end 124.333 69.46) (width 0.5) (layer "F.Cu") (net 13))
 (segment (start 124.46 67.056) (end 124.333 67.183) (width 0.5) (layer "F.Cu") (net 13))
 (segment (start 132.08 65.532) (end 129.54 68.072) (width 0.5) (layer "F.Cu") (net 13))
 (segment (start 132.08 64.516) (end 132.08 65.532) (width 0.5) (layer "F.Cu") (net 13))
 (via (at 128.524 68.072) (size 1) (drill 0.5) (layers "F.Cu" "B.Cu") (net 13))
 (via (at 124.46 67.056) (size 1) (drill 0.5) (layers "F.Cu" "B.Cu") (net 13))
 (via (at 132.08 64.516) (size 1) (drill 0.5) (layers "F.Cu" "B.Cu") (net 13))
 (segment (start 128.524 68.072) (end 125.476 68.072) (width 0.5) (layer "B.Cu") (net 13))
 (segment (start 142.245 54.351) (end 132.08 64.516) (width 0.5) (layer "B.Cu") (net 13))
 (segment (start 144.78 54.351) (end 142.245 54.351) (width 0.5) (layer "B.Cu") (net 13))
 (segment (start 125.476 68.072) (end 124.46 67.056) (width 0.5) (layer "B.Cu") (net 13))
 (segment (start 132.08 62.484) (end 129.159 65.405) (width 0.5) (layer "F.Cu") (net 14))
 (segment (start 129.159 65.405) (end 126.603 65.405) (width 0.5) (layer "F.Cu") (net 14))
 (via (at 132.08 62.484) (size 1) (drill 0.5) (layers "F.Cu" "B.Cu") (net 14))
 (segment (start 132.588 61.976) (end 132.08 62.484) (width 0.5) (layer "B.Cu") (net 14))
 (segment (start 144.78 51.811) (end 142.753 51.811) (width 0.5) (layer "B.Cu") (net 14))
 (segment (start 142.753 51.811) (end 132.588 61.976) (width 0.5) (layer "B.Cu") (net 14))
 (segment (start 130.053 47.747) (end 130.053 43.18) (width 0.5) (layer "F.Cu") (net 19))
 (segment (start 128.016 49.784) (end 130.053 47.747) (width 0.5) (layer "F.Cu") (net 19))
 (segment (start 120.429 49.784) (end 128.016 49.784) (width 0.5) (layer "F.Cu") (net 19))
 (segment (start 119.253 52.46) (end 119.253 50.96) (width 0.5) (layer "F.Cu") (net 19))
 (segment (start 119.253 50.96) (end 120.429 49.784) (width 0.5) (layer "F.Cu") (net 19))
 (segment (start 121.793 53.915738) (end 121.793 52.46) (width 0.5) (layer "F.Cu") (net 20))
 (segment (start 121.382369 54.326369) (end 121.793 53.915738) (width 0.5) (layer "F.Cu") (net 20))
 (via (at 121.382369 54.326369) (size 1) (drill 0.5) (layers "F.Cu" "B.Cu") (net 20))
 (segment (start 122.457631 54.326369) (end 132.593 44.191) (width 0.5) (layer "B.Cu") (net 20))
 (segment (start 121.382369 54.326369) (end 122.457631 54.326369) (width 0.5) (layer "B.Cu") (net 20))
 (segment (start 132.593 44.191) (end 132.593 43.18) (width 0.5) (layer "B.Cu") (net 20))
 (segment (start 121.930861 55.393122) (end 122.032645 55.393122) (width 0.5) (layer "F.Cu") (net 21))
 (segment (start 122.032645 55.393122) (end 123.063 54.362767) (width 0.5) (layer "F.Cu") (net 21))
 (segment (start 123.063 54.362767) (end 123.063 52.46) (width 0.5) (layer "F.Cu") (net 21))
 (via (at 121.930861 55.393122) (size 1) (drill 0.5) (layers "F.Cu" "B.Cu") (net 21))
 (segment (start 121.930861 55.393122) (end 122.588066 55.393122) (width 0.5) (layer "B.Cu") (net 21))
 (segment (start 134.801188 43.18) (end 135.133 43.18) (width 0.5) (layer "B.Cu") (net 21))
 (segment (start 122.588066 55.393122) (end 134.801188 43.18) (width 0.5) (layer "B.Cu") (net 21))
 (segment (start 111.633 52.46) (end 111.633 50.419) (width 0.5) (layer "F.Cu") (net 43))
 (segment (start 111.633 50.419) (end 111.76 50.292) (width 0.5) (layer "F.Cu") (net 43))
 (via (at 111.76 50.292) (size 0.8) (drill 0.4) (layers "F.Cu" "B.Cu") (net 43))
 (segment (start 112.268 49.784) (end 119.111 49.784) (width 0.5) (layer "B.Cu") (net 43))
 (segment (start 119.111 49.784) (end 121.168 47.727) (width 0.5) (layer "B.Cu") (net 43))
 (segment (start 111.76 50.292) (end 112.268 49.784) (width 0.5) (layer "B.Cu") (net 43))
 (segment (start 115.443 52.46) (end 115.443 48.133) (width 0.5) (layer "F.Cu") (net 42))
 (segment (start 115.443 48.133) (end 116.332 47.244) (width 0.5) (layer "F.Cu") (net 42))
 (via (at 116.332 47.244) (size 0.8) (drill 0.4) (layers "F.Cu" "B.Cu") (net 42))
 (segment (start 121.92 45.72) (end 123.708 47.508) (width 0.5) (layer "B.Cu") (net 42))
 (segment (start 123.708 47.508) (end 123.708 47.727) (width 0.5) (layer "B.Cu") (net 42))
 (segment (start 116.332 47.244) (end 117.856 45.72) (width 0.5) (layer "B.Cu") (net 42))
 (segment (start 117.856 45.72) (end 121.92 45.72) (width 0.5) (layer "B.Cu") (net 42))
 (segment (start 112.903 52.46) (end 112.903 43.526) (width 0.5) (layer "F.Cu") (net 9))
 (segment (start 112.903 43.526) (end 112.532 43.155) (width 0.5) (layer "F.Cu") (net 9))
 (segment (start 114.173 44.054) (end 115.072 43.155) (width 0.5) (layer "F.Cu") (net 10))
 (segment (start 114.173 52.46) (end 114.173 44.054) (width 0.5) (layer "F.Cu") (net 10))
 (segment (start 138.034 74.676) (end 138.034 76.85) (width 0.35) (layer "B.Cu") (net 45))
 (segment (start 138.034 76.85) (end 137.668 77.216) (width 0.35) (layer "B.Cu") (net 45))
 (segment (start 132.62 69.596) (end 132.484 69.46) (width 0.35) (layer "F.Cu") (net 32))
 (segment (start 132.484 69.46) (end 125.603 69.46) (width 0.35) (layer "F.Cu") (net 32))
 (segment (start 136.017 50.865) (end 136.017 52.451) (width 0.5) (layer "F.Cu") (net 16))
 (segment (start 122.936 56.388) (end 123.952 56.388) (width 0.5) (layer "F.Cu") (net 16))
 (segment (start 134.62 53.848) (end 129.54 53.848) (width 0.5) (layer "F.Cu") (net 16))
 (segment (start 123.952 56.388) (end 124.46 55.88) (width 0.5) (layer "F.Cu") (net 16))
 (segment (start 124.46 55.88) (end 124.46 52.587) (width 0.5) (layer "F.Cu") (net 16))
 (segment (start 129.54 53.848) (end 129.032 53.34) (width 0.5) (layer "F.Cu") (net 16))
 (segment (start 124.46 52.587) (end 124.333 52.46) (width 0.5) (layer "F.Cu") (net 16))
 (segment (start 136.017 52.451) (end 134.62 53.848) (width 0.5) (layer "F.Cu") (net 16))
 (via (at 129.032 53.34) (size 1) (drill 0.5) (layers "F.Cu" "B.Cu") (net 16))
 (via (at 122.936 56.388) (size 1) (drill 0.5) (layers "F.Cu" "B.Cu") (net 16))
 (segment (start 129.032 53.34) (end 125.984 56.388) (width 0.5) (layer "B.Cu") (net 16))
 (segment (start 125.984 56.388) (end 122.936 56.388) (width 0.5) (layer "B.Cu") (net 16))
 (segment (start 120.523 52.46) (end 120.523 50.96) (width 0.5) (layer "F.Cu") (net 17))
 (segment (start 120.523 50.96) (end 120.99948 50.48352) (width 0.5) (layer "F.Cu") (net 17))
 (segment (start 132.207 48.895) (end 132.207 50.865) (width 0.5) (layer "F.Cu") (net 17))
 (segment (start 131.572 48.26) (end 132.207 48.895) (width 0.5) (layer "F.Cu") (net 17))
 (segment (start 120.99948 50.48352) (end 128.305751 50.483519) (width 0.5) (layer "F.Cu") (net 17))
 (segment (start 128.305751 50.483519) (end 130.52927 48.26) (width 0.5) (layer "F.Cu") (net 17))
 (segment (start 130.52927 48.26) (end 131.572 48.26) (width 0.5) (layer "F.Cu") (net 17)))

